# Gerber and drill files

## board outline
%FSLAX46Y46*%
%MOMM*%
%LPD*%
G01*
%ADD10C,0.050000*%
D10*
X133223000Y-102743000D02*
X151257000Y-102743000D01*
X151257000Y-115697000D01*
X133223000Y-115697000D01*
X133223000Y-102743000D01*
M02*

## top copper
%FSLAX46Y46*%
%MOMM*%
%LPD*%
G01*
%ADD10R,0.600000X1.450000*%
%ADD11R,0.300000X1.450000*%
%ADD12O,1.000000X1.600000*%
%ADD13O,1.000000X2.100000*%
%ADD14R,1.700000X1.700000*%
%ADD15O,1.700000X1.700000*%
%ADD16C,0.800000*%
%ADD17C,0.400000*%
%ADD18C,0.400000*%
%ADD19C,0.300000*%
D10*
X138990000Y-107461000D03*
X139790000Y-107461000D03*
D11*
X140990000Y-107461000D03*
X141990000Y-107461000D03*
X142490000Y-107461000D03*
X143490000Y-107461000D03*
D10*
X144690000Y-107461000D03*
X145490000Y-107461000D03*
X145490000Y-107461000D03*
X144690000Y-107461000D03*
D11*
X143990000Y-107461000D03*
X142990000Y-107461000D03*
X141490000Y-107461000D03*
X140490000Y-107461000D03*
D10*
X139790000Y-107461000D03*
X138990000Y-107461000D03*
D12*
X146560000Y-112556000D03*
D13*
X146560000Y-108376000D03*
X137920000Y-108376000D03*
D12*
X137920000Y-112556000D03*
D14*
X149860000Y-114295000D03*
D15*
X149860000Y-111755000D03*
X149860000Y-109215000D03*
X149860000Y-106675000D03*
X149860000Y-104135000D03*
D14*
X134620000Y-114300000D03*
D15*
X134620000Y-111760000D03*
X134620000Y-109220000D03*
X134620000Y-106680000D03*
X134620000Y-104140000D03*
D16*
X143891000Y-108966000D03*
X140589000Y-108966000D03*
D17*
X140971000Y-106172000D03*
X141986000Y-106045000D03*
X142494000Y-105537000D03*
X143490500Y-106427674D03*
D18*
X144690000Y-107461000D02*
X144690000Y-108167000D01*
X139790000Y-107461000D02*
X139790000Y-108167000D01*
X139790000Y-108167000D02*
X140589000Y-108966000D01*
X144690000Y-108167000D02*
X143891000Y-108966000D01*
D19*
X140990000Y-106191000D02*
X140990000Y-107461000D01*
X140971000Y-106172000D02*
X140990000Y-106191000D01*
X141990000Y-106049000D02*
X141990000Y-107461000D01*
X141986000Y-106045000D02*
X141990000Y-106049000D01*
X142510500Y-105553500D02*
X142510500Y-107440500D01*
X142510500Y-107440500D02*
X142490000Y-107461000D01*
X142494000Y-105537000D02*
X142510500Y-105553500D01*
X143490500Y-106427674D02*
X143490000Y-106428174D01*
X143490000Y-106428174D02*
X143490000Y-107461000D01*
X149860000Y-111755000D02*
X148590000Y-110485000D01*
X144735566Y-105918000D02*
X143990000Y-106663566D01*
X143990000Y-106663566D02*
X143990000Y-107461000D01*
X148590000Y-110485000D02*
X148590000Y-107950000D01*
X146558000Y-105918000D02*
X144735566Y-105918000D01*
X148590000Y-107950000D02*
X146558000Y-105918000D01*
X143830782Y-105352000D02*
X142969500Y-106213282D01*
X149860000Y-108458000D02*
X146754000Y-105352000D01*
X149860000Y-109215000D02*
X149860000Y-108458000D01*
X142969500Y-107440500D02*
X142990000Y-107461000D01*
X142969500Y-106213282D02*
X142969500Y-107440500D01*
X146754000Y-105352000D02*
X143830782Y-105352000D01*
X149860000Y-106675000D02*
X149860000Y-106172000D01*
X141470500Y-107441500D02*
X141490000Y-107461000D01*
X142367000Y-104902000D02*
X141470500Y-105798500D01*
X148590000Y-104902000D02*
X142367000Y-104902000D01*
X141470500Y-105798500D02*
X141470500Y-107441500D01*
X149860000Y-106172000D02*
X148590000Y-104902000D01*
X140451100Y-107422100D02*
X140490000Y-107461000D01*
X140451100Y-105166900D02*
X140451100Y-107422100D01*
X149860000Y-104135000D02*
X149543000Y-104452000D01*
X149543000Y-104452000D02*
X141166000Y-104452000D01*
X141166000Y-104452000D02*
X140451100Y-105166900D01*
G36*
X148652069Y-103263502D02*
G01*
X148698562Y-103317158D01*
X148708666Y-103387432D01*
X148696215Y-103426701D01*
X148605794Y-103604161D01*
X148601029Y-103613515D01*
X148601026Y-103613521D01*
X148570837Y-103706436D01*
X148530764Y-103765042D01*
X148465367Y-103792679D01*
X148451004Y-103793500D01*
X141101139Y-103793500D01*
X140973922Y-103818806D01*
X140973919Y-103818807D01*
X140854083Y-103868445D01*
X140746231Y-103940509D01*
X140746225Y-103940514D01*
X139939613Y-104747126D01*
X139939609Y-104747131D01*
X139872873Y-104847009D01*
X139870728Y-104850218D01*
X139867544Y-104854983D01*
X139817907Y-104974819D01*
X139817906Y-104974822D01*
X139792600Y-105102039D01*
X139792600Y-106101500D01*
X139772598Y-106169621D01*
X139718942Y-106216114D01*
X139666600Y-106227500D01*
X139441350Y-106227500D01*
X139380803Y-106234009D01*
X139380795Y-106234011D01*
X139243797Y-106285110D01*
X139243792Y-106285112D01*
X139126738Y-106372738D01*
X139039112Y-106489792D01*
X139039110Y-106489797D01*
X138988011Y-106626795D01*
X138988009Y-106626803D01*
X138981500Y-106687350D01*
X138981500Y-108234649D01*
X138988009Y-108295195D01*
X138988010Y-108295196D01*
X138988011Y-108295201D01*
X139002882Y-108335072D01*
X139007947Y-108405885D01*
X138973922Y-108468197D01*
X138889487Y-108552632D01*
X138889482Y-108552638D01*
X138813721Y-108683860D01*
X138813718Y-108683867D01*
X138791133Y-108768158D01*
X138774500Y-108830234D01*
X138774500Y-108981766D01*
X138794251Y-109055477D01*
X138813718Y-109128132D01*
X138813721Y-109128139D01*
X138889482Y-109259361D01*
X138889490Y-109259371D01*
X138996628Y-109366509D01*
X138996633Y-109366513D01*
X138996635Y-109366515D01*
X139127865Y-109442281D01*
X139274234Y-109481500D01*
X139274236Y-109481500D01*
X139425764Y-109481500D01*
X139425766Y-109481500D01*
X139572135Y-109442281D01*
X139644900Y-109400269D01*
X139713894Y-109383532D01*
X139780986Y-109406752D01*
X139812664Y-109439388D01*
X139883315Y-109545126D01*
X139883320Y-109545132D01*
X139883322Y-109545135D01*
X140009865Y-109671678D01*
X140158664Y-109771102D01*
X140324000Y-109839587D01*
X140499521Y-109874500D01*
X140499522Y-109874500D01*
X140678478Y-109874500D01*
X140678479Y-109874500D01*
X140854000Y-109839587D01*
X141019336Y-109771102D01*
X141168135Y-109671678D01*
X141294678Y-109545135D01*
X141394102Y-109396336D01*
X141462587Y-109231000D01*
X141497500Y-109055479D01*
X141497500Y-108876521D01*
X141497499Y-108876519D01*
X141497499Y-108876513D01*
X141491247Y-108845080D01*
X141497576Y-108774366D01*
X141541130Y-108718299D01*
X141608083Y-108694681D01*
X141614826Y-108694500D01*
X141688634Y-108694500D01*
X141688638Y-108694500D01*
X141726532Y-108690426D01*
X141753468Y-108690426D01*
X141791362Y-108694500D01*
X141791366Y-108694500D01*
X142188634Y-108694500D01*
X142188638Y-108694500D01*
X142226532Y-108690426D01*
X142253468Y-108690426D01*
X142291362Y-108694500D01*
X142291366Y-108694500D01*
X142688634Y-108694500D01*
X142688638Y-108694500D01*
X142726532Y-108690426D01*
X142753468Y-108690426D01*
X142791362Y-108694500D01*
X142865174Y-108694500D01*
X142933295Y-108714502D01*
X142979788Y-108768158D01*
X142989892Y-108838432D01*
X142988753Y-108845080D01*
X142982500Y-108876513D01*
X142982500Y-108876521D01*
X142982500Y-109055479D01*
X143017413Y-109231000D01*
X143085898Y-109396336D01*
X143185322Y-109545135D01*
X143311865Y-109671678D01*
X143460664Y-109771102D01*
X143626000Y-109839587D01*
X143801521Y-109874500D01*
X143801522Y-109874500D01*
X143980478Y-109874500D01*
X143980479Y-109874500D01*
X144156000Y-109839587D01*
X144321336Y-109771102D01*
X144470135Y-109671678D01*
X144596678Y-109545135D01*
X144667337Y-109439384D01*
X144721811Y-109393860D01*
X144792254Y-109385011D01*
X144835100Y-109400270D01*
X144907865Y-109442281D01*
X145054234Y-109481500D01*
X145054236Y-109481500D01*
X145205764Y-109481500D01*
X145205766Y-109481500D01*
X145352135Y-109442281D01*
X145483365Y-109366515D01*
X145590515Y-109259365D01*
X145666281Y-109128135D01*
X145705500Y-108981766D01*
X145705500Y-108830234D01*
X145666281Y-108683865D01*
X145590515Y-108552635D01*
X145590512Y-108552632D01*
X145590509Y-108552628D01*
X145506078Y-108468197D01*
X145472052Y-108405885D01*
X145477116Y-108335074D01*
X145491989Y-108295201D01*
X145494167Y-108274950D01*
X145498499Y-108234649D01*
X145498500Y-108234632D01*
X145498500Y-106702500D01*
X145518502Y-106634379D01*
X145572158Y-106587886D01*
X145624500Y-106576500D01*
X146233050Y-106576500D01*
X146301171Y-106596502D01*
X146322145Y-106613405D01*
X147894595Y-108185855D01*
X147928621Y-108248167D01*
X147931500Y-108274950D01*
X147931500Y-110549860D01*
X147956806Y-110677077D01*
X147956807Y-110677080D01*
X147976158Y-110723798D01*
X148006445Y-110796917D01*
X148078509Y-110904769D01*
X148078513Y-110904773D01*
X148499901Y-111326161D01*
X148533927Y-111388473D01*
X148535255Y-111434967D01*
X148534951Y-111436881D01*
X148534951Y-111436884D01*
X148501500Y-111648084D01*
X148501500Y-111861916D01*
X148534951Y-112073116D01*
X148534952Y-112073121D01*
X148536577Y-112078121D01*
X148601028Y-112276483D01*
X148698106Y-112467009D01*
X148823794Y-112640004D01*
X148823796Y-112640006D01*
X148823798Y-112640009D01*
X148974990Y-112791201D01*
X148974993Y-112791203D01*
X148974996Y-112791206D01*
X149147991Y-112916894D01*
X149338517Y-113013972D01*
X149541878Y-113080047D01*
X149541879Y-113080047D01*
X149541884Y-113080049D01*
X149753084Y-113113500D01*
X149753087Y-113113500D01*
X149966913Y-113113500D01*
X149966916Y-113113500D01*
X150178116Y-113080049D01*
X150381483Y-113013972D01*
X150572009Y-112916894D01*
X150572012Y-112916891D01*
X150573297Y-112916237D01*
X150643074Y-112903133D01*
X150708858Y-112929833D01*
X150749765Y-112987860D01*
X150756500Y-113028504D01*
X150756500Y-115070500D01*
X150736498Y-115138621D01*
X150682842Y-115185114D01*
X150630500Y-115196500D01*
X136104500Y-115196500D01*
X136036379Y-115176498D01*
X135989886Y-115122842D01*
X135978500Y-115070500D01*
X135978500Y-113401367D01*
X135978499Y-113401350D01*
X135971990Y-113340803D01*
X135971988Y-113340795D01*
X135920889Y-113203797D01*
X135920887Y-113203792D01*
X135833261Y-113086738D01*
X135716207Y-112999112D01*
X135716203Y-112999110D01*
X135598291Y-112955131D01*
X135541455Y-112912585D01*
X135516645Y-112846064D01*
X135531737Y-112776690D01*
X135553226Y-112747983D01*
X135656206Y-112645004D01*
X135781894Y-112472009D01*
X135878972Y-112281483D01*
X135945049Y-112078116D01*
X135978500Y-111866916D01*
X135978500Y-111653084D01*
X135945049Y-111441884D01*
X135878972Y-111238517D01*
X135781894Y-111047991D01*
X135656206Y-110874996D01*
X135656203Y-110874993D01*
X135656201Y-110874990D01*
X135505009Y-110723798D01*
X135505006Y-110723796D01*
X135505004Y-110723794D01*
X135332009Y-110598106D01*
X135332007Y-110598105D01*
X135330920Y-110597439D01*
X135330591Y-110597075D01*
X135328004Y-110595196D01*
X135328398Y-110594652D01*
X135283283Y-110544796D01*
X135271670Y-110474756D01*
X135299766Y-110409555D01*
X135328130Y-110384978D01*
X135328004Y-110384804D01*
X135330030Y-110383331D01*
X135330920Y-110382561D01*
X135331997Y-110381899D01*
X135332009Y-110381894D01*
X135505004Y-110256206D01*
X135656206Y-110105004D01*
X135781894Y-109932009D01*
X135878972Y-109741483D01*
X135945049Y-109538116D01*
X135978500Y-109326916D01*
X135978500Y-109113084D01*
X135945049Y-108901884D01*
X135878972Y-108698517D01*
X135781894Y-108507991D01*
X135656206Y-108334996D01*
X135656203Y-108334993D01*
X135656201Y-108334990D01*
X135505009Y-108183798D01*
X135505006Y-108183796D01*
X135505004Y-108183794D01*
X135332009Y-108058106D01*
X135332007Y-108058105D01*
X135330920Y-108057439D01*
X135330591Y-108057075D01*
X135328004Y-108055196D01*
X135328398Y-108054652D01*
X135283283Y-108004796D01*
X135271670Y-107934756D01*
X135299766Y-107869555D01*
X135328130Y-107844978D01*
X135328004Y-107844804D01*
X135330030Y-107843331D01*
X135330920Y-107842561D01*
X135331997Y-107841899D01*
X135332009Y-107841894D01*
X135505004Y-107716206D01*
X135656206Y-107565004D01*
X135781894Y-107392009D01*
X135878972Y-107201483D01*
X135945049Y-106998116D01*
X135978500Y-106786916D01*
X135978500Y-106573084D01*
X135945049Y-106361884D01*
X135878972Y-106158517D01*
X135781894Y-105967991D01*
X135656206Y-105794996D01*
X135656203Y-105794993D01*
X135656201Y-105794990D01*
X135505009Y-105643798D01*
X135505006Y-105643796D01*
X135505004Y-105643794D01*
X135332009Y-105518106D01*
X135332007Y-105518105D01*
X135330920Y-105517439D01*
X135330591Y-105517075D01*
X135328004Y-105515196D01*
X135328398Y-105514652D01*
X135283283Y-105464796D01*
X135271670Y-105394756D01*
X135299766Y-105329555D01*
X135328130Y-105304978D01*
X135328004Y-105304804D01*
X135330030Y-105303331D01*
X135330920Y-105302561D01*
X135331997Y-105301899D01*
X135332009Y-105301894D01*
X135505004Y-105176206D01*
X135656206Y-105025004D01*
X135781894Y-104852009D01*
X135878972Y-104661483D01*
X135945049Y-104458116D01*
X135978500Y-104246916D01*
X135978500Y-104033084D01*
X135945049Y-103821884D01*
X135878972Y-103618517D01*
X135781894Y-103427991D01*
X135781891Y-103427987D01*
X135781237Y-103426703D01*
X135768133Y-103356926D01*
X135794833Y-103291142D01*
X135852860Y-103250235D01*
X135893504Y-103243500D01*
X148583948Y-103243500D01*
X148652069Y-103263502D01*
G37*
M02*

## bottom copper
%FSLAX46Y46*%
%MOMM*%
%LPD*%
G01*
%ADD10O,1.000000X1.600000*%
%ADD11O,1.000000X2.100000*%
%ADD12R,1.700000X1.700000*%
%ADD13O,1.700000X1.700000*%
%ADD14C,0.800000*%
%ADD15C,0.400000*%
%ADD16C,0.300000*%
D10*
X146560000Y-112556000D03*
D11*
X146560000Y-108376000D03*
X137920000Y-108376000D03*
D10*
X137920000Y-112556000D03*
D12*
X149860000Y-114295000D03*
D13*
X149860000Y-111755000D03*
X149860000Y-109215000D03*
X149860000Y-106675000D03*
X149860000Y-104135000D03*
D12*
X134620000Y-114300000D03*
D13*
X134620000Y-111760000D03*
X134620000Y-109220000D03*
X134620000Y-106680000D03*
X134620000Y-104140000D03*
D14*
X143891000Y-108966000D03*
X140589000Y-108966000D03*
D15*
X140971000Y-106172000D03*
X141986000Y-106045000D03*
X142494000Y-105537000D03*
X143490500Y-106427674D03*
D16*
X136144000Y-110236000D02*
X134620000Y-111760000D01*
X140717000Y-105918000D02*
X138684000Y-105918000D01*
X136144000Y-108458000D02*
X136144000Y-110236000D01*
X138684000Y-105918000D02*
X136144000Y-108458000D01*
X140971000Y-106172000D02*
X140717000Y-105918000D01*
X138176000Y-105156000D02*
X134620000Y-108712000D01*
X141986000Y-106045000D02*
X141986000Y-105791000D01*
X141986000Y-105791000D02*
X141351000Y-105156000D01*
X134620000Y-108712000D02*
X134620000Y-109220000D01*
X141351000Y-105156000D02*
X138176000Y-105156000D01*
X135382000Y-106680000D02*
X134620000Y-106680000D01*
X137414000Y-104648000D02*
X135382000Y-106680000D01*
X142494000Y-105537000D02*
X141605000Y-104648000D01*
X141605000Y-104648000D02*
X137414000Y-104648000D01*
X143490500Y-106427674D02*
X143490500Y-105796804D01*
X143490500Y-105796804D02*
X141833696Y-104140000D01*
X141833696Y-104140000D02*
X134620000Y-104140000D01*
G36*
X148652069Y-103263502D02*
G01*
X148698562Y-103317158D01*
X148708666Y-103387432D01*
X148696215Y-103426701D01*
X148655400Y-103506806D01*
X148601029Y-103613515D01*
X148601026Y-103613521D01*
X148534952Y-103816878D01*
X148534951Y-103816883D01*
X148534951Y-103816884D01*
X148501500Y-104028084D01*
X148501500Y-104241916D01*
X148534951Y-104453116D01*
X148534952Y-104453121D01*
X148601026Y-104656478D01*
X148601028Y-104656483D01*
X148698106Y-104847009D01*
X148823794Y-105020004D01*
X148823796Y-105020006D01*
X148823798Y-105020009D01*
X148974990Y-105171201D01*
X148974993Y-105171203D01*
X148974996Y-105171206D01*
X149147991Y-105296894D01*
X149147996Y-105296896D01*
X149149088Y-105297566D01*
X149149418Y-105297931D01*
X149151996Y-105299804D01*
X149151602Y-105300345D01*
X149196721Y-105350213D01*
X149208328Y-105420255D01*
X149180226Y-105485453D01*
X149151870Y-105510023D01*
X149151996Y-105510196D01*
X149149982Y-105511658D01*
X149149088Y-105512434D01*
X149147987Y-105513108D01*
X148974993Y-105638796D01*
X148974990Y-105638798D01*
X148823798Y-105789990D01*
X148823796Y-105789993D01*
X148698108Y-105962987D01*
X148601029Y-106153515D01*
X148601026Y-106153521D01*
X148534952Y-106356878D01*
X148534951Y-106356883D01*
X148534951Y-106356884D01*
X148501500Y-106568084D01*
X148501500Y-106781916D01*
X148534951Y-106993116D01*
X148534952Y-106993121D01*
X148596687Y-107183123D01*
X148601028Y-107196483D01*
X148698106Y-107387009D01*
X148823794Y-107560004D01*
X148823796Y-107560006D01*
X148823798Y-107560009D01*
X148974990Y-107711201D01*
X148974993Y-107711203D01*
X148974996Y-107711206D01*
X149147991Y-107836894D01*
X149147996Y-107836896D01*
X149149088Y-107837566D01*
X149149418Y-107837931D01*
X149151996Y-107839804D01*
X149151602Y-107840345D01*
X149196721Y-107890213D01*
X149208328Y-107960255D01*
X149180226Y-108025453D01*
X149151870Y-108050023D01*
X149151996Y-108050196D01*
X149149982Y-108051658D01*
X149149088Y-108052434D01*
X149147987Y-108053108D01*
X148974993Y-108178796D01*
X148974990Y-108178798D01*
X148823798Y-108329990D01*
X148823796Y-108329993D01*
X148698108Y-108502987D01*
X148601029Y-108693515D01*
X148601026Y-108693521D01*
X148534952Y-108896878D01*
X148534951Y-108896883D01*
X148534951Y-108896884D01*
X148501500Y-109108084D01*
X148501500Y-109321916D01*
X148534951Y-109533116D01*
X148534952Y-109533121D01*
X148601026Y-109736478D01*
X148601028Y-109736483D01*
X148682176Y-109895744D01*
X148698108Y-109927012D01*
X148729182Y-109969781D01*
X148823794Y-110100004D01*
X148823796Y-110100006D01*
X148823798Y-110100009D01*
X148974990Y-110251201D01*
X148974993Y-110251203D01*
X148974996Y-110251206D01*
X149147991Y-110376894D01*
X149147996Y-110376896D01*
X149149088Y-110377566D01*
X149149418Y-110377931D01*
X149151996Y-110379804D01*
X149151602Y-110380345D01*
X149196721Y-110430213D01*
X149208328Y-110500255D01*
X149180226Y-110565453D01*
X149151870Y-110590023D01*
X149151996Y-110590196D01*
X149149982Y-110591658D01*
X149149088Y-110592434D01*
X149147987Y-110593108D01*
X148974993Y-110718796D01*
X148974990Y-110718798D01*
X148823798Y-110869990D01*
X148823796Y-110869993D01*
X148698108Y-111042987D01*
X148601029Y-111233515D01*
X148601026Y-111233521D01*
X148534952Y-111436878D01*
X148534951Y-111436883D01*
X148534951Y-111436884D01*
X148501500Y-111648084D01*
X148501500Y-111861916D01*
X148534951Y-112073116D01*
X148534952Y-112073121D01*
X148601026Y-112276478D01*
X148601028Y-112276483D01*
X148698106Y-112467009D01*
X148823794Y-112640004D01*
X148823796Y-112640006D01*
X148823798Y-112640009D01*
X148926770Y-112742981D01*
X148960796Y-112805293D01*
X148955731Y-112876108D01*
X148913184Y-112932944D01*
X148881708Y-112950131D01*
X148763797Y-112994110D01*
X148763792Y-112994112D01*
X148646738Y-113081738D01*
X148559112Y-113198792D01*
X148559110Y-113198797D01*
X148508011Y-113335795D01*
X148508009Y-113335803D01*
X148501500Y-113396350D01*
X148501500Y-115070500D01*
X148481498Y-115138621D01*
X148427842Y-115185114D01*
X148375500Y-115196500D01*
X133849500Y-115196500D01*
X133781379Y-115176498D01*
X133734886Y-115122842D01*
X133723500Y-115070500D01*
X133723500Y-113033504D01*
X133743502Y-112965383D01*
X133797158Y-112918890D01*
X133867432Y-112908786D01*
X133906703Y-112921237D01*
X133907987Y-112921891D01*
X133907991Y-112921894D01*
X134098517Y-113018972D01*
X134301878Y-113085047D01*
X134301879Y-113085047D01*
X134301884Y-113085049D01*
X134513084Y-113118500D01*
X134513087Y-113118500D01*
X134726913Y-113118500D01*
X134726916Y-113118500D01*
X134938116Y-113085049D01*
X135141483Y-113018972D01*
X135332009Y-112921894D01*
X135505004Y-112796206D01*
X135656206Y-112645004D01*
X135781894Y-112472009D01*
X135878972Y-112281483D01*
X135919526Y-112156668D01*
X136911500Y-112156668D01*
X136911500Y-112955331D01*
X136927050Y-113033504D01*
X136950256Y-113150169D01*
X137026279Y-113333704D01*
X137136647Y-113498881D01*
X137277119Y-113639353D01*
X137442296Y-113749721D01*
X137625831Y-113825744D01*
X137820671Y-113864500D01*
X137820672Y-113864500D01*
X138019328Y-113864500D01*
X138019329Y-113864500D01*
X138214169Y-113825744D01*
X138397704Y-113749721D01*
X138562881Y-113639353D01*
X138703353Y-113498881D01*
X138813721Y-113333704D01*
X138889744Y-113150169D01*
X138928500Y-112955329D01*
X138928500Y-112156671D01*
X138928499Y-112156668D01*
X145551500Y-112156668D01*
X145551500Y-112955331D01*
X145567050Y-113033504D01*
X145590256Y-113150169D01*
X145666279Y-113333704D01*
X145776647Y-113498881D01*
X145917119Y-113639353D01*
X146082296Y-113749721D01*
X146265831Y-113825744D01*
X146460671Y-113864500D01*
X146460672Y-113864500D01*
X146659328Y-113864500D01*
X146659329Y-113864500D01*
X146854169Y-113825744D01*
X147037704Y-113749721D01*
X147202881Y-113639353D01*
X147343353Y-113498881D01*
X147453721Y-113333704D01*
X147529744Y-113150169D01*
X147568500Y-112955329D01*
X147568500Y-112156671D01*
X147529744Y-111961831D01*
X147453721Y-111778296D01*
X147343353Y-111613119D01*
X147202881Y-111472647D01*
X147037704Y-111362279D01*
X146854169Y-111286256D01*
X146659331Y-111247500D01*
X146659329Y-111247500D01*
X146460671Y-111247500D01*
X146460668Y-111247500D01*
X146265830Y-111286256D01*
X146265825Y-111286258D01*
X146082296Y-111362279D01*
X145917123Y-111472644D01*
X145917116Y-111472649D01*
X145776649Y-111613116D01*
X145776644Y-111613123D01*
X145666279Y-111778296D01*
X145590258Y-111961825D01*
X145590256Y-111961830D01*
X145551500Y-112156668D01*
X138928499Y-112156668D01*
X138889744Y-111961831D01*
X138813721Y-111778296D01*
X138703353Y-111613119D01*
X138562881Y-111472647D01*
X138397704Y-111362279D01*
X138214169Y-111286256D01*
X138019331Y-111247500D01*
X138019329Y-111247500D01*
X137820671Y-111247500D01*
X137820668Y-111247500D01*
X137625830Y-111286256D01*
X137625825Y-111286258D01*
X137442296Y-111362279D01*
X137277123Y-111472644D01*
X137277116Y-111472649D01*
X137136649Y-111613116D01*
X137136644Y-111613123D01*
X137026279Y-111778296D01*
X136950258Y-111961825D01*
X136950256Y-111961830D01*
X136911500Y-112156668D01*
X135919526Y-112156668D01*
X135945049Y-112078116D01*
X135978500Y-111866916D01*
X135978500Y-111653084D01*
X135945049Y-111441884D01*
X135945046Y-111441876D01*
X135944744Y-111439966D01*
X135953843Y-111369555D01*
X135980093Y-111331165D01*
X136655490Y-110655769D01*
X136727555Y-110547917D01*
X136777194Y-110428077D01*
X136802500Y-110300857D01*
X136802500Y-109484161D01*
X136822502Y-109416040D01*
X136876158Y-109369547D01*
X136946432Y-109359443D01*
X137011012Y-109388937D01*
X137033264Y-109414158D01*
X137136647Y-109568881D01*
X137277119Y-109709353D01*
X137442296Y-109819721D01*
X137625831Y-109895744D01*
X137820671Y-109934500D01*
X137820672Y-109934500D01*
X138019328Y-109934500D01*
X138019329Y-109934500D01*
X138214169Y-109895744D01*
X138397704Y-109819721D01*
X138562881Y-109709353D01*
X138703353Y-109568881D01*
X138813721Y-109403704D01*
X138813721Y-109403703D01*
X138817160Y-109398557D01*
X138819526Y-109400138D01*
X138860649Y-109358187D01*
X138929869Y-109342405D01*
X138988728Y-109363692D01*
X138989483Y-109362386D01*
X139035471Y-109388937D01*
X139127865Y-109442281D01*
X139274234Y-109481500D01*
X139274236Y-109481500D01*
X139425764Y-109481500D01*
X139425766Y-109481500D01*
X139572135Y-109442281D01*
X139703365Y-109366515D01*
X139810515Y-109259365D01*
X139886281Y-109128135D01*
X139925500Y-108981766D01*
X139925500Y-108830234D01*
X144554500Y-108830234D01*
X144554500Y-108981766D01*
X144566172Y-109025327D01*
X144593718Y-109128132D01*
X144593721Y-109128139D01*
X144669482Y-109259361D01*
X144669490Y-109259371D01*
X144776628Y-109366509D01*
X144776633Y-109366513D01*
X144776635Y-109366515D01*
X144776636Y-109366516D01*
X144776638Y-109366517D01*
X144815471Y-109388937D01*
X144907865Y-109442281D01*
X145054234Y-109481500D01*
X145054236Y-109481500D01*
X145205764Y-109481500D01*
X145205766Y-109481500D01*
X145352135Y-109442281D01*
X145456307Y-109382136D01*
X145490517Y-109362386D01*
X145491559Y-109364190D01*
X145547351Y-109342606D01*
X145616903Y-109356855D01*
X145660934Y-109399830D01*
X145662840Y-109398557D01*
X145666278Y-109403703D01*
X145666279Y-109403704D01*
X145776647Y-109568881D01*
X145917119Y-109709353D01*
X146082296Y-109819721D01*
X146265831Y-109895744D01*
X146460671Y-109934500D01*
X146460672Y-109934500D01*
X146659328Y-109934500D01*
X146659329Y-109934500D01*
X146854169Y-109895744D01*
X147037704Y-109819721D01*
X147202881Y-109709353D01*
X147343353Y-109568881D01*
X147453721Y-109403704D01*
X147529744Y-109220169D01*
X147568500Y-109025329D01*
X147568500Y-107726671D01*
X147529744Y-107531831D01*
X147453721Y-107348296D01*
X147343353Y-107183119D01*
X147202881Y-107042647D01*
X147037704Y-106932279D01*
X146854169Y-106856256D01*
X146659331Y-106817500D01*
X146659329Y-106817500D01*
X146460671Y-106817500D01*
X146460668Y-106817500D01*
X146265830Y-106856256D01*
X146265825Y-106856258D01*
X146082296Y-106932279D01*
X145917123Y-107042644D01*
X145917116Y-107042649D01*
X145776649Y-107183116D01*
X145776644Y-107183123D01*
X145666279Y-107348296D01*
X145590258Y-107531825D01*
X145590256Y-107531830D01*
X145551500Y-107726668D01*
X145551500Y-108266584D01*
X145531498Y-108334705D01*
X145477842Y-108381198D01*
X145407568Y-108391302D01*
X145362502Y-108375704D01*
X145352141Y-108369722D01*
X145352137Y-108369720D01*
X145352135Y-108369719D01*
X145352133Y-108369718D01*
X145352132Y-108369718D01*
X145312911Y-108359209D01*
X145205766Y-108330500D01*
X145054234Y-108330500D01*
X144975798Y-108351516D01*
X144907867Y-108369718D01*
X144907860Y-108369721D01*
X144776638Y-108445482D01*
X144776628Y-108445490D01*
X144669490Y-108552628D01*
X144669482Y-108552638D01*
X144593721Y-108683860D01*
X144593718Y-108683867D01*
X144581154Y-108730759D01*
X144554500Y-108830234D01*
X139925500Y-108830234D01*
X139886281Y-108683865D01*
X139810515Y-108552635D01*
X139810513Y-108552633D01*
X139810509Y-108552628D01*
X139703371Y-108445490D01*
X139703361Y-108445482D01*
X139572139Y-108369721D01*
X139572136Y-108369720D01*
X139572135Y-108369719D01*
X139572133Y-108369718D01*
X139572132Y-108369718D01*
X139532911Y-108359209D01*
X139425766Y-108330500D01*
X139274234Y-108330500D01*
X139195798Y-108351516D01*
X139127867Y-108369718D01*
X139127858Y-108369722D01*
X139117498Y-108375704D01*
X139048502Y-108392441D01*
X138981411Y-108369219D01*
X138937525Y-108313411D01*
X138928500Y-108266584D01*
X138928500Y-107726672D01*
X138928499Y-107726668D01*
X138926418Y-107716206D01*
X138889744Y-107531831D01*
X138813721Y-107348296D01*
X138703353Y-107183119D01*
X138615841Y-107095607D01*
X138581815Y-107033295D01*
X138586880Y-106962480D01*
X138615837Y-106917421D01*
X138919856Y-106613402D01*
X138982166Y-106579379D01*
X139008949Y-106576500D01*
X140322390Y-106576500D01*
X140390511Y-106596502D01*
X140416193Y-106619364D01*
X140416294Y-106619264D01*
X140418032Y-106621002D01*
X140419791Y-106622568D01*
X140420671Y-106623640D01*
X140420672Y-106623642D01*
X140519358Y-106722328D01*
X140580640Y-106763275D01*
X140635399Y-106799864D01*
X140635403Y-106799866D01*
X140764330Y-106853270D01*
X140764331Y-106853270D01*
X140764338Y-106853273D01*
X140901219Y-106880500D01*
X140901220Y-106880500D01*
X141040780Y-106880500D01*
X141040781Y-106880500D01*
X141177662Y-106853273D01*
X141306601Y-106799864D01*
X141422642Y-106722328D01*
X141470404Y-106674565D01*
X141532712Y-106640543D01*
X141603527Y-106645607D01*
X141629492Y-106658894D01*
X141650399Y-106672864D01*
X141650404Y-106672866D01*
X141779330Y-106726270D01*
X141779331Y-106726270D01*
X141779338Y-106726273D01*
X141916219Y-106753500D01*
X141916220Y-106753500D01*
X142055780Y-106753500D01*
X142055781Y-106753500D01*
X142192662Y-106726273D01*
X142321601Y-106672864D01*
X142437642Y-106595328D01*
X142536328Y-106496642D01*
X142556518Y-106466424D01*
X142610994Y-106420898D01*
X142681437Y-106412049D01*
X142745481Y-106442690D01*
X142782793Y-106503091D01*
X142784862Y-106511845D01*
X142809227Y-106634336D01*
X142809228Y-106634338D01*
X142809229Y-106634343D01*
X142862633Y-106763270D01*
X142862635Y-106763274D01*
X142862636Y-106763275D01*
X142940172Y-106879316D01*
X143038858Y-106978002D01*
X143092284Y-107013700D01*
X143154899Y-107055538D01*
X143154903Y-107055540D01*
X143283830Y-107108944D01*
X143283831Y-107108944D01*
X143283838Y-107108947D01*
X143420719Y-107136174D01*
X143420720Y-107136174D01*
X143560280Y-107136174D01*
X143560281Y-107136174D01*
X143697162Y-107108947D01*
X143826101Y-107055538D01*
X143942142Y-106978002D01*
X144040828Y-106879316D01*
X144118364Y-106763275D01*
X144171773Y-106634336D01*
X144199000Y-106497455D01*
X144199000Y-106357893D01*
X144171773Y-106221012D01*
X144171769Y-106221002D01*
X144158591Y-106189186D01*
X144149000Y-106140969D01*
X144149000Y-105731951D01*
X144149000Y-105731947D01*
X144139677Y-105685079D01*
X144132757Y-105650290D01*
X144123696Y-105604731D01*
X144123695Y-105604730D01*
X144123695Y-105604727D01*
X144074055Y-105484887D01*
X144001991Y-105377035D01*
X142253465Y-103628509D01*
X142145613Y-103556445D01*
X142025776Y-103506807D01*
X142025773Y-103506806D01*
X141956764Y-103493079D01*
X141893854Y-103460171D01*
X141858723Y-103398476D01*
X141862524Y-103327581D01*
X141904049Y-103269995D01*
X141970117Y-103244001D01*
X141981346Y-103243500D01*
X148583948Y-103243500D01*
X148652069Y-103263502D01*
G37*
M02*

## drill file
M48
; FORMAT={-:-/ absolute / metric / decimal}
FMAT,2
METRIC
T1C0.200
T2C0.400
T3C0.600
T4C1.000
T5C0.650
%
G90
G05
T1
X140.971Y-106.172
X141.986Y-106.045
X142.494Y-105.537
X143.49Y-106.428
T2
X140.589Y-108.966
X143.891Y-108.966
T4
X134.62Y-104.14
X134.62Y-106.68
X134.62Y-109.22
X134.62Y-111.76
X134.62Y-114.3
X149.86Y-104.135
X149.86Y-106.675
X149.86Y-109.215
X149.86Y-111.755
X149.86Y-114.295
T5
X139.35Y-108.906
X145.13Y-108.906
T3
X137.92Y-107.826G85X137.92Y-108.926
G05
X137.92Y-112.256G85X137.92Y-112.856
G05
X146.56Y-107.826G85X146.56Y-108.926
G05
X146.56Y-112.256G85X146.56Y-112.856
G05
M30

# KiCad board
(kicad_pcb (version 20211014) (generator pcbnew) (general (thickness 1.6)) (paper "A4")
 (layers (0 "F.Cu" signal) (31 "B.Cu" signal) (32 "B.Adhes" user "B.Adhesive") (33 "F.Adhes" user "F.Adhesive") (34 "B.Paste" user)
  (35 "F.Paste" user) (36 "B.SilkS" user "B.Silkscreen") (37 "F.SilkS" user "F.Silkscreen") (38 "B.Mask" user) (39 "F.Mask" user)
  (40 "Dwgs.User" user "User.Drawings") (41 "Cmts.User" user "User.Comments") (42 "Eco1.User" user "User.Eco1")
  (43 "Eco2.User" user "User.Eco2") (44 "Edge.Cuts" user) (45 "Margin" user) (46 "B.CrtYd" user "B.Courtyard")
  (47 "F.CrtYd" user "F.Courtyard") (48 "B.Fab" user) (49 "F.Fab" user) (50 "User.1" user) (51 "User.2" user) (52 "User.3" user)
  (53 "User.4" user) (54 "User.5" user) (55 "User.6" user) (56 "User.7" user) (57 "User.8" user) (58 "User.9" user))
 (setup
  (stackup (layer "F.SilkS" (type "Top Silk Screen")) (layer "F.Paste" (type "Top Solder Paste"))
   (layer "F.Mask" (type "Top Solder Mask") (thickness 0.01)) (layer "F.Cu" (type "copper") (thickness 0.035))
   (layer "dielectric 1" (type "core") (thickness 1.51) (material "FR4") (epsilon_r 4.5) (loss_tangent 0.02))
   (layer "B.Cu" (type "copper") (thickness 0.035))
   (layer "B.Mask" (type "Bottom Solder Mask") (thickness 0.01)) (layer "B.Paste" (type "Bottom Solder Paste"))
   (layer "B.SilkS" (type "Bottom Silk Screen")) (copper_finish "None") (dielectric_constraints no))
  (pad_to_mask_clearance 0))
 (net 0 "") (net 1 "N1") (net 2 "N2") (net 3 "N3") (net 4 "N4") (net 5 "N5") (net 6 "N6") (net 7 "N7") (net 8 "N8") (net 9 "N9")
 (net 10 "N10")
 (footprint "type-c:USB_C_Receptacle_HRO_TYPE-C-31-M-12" (layer "F.Cu") (at 142.24 111.506)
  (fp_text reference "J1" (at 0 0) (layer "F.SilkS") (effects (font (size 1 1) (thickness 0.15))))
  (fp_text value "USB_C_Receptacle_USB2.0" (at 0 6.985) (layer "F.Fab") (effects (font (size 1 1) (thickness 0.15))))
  (pad "" np_thru_hole circle (at -2.89 -2.6) (size 0.65 0.65) (drill 0.65) (layers *.Cu *.Mask))
  (pad "" np_thru_hole circle (at 2.89 -2.6) (size 0.65 0.65) (drill 0.65) (layers *.Cu *.Mask))
  (pad "A1" smd rect (at -3.25 -4.045) (size 0.6 1.45) (layers "F.Cu" "F.Paste" "F.Mask") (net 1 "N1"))
  (pad "A4" smd rect (at -2.45 -4.045) (size 0.6 1.45) (layers "F.Cu" "F.Paste" "F.Mask") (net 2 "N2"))
  (pad "A5" smd rect (at -1.25 -4.045) (size 0.3 1.45) (layers "F.Cu" "F.Paste" "F.Mask") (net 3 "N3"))
  (pad "A6" smd rect (at -0.25 -4.045) (size 0.3 1.45) (layers "F.Cu" "F.Paste" "F.Mask") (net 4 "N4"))
  (pad "A7" smd rect (at 0.25 -4.045) (size 0.3 1.45) (layers "F.Cu" "F.Paste" "F.Mask") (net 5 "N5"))
  (pad "A8" smd rect (at 1.25 -4.045) (size 0.3 1.45) (layers "F.Cu" "F.Paste" "F.Mask") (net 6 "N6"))
  (pad "A9" smd rect (at 2.45 -4.045) (size 0.6 1.45) (layers "F.Cu" "F.Paste" "F.Mask") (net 2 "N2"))
  (pad "A12" smd rect (at 3.25 -4.045) (size 0.6 1.45) (layers "F.Cu" "F.Paste" "F.Mask") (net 1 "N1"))
  (pad "B1" smd rect (at 3.25 -4.045) (size 0.6 1.45) (layers "F.Cu" "F.Paste" "F.Mask") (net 1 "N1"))
  (pad "B4" smd rect (at 2.45 -4.045) (size 0.6 1.45) (layers "F.Cu" "F.Paste" "F.Mask") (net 2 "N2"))
  (pad "B5" smd rect (at 1.75 -4.045) (size 0.3 1.45) (layers "F.Cu" "F.Paste" "F.Mask") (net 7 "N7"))
  (pad "B6" smd rect (at 0.75 -4.045) (size 0.3 1.45) (layers "F.Cu" "F.Paste" "F.Mask") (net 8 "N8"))
  (pad "B7" smd rect (at -0.75 -4.045) (size 0.3 1.45) (layers "F.Cu" "F.Paste" "F.Mask") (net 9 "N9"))
  (pad "B8" smd rect (at -1.75 -4.045) (size 0.3 1.45) (layers "F.Cu" "F.Paste" "F.Mask") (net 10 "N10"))
  (pad "B9" smd rect (at -2.45 -4.045) (size 0.6 1.45) (layers "F.Cu" "F.Paste" "F.Mask") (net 2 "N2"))
  (pad "B12" smd rect (at -3.25 -4.045) (size 0.6 1.45) (layers "F.Cu" "F.Paste" "F.Mask") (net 1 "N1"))
  (pad "S1" thru_hole oval (at 4.32 1.05) (size 1 1.6) (drill oval 0.6 1.2) (layers *.Cu *.Mask) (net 1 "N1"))
  (pad "S1" thru_hole oval (at 4.32 -3.13) (size 1 2.1) (drill oval 0.6 1.7) (layers *.Cu *.Mask) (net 1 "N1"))
  (pad "S1" thru_hole oval (at -4.32 -3.13) (size 1 2.1) (drill oval 0.6 1.7) (layers *.Cu *.Mask) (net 1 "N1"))
  (pad "S1" thru_hole oval (at -4.32 1.05) (size 1 1.6) (drill oval 0.6 1.2) (layers *.Cu *.Mask) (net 1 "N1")))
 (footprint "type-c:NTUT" (layer "F.Cu") (at 142.24 104.775 180)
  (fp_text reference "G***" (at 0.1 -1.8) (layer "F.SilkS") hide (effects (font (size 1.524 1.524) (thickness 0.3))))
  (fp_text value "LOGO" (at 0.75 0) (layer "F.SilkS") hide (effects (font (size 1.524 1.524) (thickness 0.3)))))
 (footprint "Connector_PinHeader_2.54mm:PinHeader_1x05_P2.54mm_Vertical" (layer "B.Cu") (at 149.86 114.295)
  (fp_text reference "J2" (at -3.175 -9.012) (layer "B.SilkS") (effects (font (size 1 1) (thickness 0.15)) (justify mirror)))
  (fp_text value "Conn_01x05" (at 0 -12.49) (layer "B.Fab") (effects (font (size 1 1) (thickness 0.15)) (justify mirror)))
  (pad "1" thru_hole rect (at 0 0) (size 1.7 1.7) (drill 1) (layers *.Cu *.Mask) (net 1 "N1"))
  (pad "2" thru_hole oval (at 0 -2.54) (size 1.7 1.7) (drill 1) (layers *.Cu *.Mask) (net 7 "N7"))
  (pad "3" thru_hole oval (at 0 -5.08) (size 1.7 1.7) (drill 1) (layers *.Cu *.Mask) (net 8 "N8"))
  (pad "4" thru_hole oval (at 0 -7.62) (size 1.7 1.7) (drill 1) (layers *.Cu *.Mask) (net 9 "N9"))
  (pad "5" thru_hole oval (at 0 -10.16) (size 1.7 1.7) (drill 1) (layers *.Cu *.Mask) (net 10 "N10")))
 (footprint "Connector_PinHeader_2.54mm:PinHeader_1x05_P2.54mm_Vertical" (layer "B.Cu") (at 134.62 114.3)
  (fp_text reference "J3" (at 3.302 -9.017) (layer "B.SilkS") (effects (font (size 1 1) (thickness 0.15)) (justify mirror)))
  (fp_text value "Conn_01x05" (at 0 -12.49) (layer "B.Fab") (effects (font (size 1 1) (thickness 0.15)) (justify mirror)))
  (pad "1" thru_hole rect (at 0 0) (size 1.7 1.7) (drill 1) (layers *.Cu *.Mask) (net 2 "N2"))
  (pad "2" thru_hole oval (at 0 -2.54) (size 1.7 1.7) (drill 1) (layers *.Cu *.Mask) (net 3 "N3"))
  (pad "3" thru_hole oval (at 0 -5.08) (size 1.7 1.7) (drill 1) (layers *.Cu *.Mask) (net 4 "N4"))
  (pad "4" thru_hole oval (at 0 -7.62) (size 1.7 1.7) (drill 1) (layers *.Cu *.Mask) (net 5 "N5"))
  (pad "5" thru_hole oval (at 0 -10.16) (size 1.7 1.7) (drill 1) (layers *.Cu *.Mask) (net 6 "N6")))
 (gr_rect (start 133.223 102.743) (end 151.257 115.697) (layer "Edge.Cuts") (width 0.05) (fill none))
 (segment (start 144.69 107.461) (end 144.69 108.167) (width 0.4) (layer "F.Cu") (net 2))
 (segment (start 139.79 107.461) (end 139.79 108.167) (width 0.4) (layer "F.Cu") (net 2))
 (segment (start 139.79 108.167) (end 140.589 108.966) (width 0.4) (layer "F.Cu") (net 2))
 (segment (start 144.69 108.167) (end 143.891 108.966) (width 0.4) (layer "F.Cu") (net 2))
 (via (at 143.891 108.966) (size 0.8) (drill 0.4) (layers "F.Cu" "B.Cu") (free) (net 2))
 (via (at 140.589 108.966) (size 0.8) (drill 0.4) (layers "F.Cu" "B.Cu") (free) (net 2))
 (segment (start 140.99 106.191) (end 140.99 107.461) (width 0.3) (layer "F.Cu") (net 3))
 (segment (start 140.971 106.172) (end 140.99 106.191) (width 0.3) (layer "F.Cu") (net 3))
 (via (at 140.971 106.172) (size 0.4) (drill 0.2) (layers "F.Cu" "B.Cu") (free) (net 3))
 (segment (start 136.144 110.236) (end 134.62 111.76) (width 0.3) (layer "B.Cu") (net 3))
 (segment (start 140.717 105.918) (end 138.684 105.918) (width 0.3) (layer "B.Cu") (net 3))
 (segment (start 136.144 108.458) (end 136.144 110.236) (width 0.3) (layer "B.Cu") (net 3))
 (segment (start 138.684 105.918) (end 136.144 108.458) (width 0.3) (layer "B.Cu") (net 3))
 (segment (start 140.971 106.172) (end 140.717 105.918) (width 0.3) (layer "B.Cu") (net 3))
 (segment (start 141.99 106.049) (end 141.99 107.461) (width 0.3) (layer "F.Cu") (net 4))
 (segment (start 141.986 106.045) (end 141.99 106.049) (width 0.3) (layer "F.Cu") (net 4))
 (via (at 141.986 106.045) (size 0.4) (drill 0.2) (layers "F.Cu" "B.Cu") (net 4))
 (segment (start 138.176 105.156) (end 134.62 108.712) (width 0.3) (layer "B.Cu") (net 4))
 (segment (start 141.986 106.045) (end 141.986 105.791) (width 0.3) (layer "B.Cu") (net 4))
 (segment (start 141.986 105.791) (end 141.351 105.156) (width 0.3) (layer "B.Cu") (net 4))
 (segment (start 134.62 108.712) (end 134.62 109.22) (width 0.3) (layer "B.Cu") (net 4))
 (segment (start 141.351 105.156) (end 138.176 105.156) (width 0.3) (layer "B.Cu") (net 4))
 (segment (start 142.5105 105.5535) (end 142.5105 107.4405) (width 0.3) (layer "F.Cu") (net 5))
 (segment (start 142.5105 107.4405) (end 142.49 107.461) (width 0.3) (layer "F.Cu") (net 5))
 (segment (start 142.494 105.537) (end 142.5105 105.5535) (width 0.3) (layer "F.Cu") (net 5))
 (via (at 142.494 105.537) (size 0.4) (drill 0.2) (layers "F.Cu" "B.Cu") (free) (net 5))
 (segment (start 135.382 106.68) (end 134.62 106.68) (width 0.3) (layer "B.Cu") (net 5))
 (segment (start 137.414 104.648) (end 135.382 106.68) (width 0.3) (layer "B.Cu") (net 5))
 (segment (start 142.494 105.537) (end 141.605 104.648) (width 0.3) (layer "B.Cu") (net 5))
 (segment (start 141.605 104.648) (end 137.414 104.648) (width 0.3) (layer "B.Cu") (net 5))
 (segment (start 143.4905 106.427674) (end 143.49 106.428174) (width 0.3) (layer "F.Cu") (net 6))
 (segment (start 143.49 106.428174) (end 143.49 107.461) (width 0.3) (layer "F.Cu") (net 6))
 (via (at 143.4905 106.427674) (size 0.4) (drill 0.2) (layers "F.Cu" "B.Cu") (free) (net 6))
 (segment (start 143.4905 106.427674) (end 143.4905 105.796804) (width 0.3) (layer "B.Cu") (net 6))
 (segment (start 143.4905 105.796804) (end 141.833696 104.14) (width 0.3) (layer "B.Cu") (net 6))
 (segment (start 141.833696 104.14) (end 134.62 104.14) (width 0.3) (layer "B.Cu") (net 6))
 (segment (start 149.86 111.755) (end 148.59 110.485) (width 0.3) (layer "F.Cu") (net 7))
 (segment (start 144.735566 105.918) (end 143.99 106.663566) (width 0.3) (layer "F.Cu") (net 7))
 (segment (start 143.99 106.663566) (end 143.99 107.461) (width 0.3) (layer "F.Cu") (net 7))
 (segment (start 148.59 110.485) (end 148.59 107.95) (width 0.3) (layer "F.Cu") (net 7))
 (segment (start 146.558 105.918) (end 144.735566 105.918) (width 0.3) (layer "F.Cu") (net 7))
 (segment (start 148.59 107.95) (end 146.558 105.918) (width 0.3) (layer "F.Cu") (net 7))
 (segment (start 143.830782 105.352) (end 142.9695 106.213282) (width 0.3) (layer "F.Cu") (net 8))
 (segment (start 149.86 108.458) (end 146.754 105.352) (width 0.3) (layer "F.Cu") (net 8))
 (segment (start 149.86 109.215) (end 149.86 108.458) (width 0.3) (layer "F.Cu") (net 8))
 (segment (start 142.9695 107.4405) (end 142.99 107.461) (width 0.3) (layer "F.Cu") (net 8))
 (segment (start 142.9695 106.213282) (end 142.9695 107.4405) (width 0.3) (layer "F.Cu") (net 8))
 (segment (start 146.754 105.352) (end 143.830782 105.352) (width 0.3) (layer "F.Cu") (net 8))
 (segment (start 149.86 106.675) (end 149.86 106.172) (width 0.3) (layer "F.Cu") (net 9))
 (segment (start 141.4705 107.4415) (end 141.49 107.461) (width 0.3) (layer "F.Cu") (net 9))
 (segment (start 142.367 104.902) (end 141.4705 105.7985) (width 0.3) (layer "F.Cu") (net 9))
 (segment (start 148.59 104.902) (end 142.367 104.902) (width 0.3) (layer "F.Cu") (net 9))
 (segment (start 141.4705 105.7985) (end 141.4705 107.4415) (width 0.3) (layer "F.Cu") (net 9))
 (segment (start 149.86 106.172) (end 148.59 104.902) (width 0.3) (layer "F.Cu") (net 9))
 (segment (start 140.4511 107.4221) (end 140.49 107.461) (width 0.3) (layer "F.Cu") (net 10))
 (segment (start 140.4511 105.1669) (end 140.4511 107.4221) (width 0.3) (layer "F.Cu") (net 10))
 (segment (start 149.86 104.135) (end 149.543 104.452) (width 0.3) (layer "F.Cu") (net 10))
 (segment (start 149.543 104.452) (end 141.166 104.452) (width 0.3) (layer "F.Cu") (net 10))
 (segment (start 141.166 104.452) (end 140.4511 105.1669) (width 0.3) (layer "F.Cu") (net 10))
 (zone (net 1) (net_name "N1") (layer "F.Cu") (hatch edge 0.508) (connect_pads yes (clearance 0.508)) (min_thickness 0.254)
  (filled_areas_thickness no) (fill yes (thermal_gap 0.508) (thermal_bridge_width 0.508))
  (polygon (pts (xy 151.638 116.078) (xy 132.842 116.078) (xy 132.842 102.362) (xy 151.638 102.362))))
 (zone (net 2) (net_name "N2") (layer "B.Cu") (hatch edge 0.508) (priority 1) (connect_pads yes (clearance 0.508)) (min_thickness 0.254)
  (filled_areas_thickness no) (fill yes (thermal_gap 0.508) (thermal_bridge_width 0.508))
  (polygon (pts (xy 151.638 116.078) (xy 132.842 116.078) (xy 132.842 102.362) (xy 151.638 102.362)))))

